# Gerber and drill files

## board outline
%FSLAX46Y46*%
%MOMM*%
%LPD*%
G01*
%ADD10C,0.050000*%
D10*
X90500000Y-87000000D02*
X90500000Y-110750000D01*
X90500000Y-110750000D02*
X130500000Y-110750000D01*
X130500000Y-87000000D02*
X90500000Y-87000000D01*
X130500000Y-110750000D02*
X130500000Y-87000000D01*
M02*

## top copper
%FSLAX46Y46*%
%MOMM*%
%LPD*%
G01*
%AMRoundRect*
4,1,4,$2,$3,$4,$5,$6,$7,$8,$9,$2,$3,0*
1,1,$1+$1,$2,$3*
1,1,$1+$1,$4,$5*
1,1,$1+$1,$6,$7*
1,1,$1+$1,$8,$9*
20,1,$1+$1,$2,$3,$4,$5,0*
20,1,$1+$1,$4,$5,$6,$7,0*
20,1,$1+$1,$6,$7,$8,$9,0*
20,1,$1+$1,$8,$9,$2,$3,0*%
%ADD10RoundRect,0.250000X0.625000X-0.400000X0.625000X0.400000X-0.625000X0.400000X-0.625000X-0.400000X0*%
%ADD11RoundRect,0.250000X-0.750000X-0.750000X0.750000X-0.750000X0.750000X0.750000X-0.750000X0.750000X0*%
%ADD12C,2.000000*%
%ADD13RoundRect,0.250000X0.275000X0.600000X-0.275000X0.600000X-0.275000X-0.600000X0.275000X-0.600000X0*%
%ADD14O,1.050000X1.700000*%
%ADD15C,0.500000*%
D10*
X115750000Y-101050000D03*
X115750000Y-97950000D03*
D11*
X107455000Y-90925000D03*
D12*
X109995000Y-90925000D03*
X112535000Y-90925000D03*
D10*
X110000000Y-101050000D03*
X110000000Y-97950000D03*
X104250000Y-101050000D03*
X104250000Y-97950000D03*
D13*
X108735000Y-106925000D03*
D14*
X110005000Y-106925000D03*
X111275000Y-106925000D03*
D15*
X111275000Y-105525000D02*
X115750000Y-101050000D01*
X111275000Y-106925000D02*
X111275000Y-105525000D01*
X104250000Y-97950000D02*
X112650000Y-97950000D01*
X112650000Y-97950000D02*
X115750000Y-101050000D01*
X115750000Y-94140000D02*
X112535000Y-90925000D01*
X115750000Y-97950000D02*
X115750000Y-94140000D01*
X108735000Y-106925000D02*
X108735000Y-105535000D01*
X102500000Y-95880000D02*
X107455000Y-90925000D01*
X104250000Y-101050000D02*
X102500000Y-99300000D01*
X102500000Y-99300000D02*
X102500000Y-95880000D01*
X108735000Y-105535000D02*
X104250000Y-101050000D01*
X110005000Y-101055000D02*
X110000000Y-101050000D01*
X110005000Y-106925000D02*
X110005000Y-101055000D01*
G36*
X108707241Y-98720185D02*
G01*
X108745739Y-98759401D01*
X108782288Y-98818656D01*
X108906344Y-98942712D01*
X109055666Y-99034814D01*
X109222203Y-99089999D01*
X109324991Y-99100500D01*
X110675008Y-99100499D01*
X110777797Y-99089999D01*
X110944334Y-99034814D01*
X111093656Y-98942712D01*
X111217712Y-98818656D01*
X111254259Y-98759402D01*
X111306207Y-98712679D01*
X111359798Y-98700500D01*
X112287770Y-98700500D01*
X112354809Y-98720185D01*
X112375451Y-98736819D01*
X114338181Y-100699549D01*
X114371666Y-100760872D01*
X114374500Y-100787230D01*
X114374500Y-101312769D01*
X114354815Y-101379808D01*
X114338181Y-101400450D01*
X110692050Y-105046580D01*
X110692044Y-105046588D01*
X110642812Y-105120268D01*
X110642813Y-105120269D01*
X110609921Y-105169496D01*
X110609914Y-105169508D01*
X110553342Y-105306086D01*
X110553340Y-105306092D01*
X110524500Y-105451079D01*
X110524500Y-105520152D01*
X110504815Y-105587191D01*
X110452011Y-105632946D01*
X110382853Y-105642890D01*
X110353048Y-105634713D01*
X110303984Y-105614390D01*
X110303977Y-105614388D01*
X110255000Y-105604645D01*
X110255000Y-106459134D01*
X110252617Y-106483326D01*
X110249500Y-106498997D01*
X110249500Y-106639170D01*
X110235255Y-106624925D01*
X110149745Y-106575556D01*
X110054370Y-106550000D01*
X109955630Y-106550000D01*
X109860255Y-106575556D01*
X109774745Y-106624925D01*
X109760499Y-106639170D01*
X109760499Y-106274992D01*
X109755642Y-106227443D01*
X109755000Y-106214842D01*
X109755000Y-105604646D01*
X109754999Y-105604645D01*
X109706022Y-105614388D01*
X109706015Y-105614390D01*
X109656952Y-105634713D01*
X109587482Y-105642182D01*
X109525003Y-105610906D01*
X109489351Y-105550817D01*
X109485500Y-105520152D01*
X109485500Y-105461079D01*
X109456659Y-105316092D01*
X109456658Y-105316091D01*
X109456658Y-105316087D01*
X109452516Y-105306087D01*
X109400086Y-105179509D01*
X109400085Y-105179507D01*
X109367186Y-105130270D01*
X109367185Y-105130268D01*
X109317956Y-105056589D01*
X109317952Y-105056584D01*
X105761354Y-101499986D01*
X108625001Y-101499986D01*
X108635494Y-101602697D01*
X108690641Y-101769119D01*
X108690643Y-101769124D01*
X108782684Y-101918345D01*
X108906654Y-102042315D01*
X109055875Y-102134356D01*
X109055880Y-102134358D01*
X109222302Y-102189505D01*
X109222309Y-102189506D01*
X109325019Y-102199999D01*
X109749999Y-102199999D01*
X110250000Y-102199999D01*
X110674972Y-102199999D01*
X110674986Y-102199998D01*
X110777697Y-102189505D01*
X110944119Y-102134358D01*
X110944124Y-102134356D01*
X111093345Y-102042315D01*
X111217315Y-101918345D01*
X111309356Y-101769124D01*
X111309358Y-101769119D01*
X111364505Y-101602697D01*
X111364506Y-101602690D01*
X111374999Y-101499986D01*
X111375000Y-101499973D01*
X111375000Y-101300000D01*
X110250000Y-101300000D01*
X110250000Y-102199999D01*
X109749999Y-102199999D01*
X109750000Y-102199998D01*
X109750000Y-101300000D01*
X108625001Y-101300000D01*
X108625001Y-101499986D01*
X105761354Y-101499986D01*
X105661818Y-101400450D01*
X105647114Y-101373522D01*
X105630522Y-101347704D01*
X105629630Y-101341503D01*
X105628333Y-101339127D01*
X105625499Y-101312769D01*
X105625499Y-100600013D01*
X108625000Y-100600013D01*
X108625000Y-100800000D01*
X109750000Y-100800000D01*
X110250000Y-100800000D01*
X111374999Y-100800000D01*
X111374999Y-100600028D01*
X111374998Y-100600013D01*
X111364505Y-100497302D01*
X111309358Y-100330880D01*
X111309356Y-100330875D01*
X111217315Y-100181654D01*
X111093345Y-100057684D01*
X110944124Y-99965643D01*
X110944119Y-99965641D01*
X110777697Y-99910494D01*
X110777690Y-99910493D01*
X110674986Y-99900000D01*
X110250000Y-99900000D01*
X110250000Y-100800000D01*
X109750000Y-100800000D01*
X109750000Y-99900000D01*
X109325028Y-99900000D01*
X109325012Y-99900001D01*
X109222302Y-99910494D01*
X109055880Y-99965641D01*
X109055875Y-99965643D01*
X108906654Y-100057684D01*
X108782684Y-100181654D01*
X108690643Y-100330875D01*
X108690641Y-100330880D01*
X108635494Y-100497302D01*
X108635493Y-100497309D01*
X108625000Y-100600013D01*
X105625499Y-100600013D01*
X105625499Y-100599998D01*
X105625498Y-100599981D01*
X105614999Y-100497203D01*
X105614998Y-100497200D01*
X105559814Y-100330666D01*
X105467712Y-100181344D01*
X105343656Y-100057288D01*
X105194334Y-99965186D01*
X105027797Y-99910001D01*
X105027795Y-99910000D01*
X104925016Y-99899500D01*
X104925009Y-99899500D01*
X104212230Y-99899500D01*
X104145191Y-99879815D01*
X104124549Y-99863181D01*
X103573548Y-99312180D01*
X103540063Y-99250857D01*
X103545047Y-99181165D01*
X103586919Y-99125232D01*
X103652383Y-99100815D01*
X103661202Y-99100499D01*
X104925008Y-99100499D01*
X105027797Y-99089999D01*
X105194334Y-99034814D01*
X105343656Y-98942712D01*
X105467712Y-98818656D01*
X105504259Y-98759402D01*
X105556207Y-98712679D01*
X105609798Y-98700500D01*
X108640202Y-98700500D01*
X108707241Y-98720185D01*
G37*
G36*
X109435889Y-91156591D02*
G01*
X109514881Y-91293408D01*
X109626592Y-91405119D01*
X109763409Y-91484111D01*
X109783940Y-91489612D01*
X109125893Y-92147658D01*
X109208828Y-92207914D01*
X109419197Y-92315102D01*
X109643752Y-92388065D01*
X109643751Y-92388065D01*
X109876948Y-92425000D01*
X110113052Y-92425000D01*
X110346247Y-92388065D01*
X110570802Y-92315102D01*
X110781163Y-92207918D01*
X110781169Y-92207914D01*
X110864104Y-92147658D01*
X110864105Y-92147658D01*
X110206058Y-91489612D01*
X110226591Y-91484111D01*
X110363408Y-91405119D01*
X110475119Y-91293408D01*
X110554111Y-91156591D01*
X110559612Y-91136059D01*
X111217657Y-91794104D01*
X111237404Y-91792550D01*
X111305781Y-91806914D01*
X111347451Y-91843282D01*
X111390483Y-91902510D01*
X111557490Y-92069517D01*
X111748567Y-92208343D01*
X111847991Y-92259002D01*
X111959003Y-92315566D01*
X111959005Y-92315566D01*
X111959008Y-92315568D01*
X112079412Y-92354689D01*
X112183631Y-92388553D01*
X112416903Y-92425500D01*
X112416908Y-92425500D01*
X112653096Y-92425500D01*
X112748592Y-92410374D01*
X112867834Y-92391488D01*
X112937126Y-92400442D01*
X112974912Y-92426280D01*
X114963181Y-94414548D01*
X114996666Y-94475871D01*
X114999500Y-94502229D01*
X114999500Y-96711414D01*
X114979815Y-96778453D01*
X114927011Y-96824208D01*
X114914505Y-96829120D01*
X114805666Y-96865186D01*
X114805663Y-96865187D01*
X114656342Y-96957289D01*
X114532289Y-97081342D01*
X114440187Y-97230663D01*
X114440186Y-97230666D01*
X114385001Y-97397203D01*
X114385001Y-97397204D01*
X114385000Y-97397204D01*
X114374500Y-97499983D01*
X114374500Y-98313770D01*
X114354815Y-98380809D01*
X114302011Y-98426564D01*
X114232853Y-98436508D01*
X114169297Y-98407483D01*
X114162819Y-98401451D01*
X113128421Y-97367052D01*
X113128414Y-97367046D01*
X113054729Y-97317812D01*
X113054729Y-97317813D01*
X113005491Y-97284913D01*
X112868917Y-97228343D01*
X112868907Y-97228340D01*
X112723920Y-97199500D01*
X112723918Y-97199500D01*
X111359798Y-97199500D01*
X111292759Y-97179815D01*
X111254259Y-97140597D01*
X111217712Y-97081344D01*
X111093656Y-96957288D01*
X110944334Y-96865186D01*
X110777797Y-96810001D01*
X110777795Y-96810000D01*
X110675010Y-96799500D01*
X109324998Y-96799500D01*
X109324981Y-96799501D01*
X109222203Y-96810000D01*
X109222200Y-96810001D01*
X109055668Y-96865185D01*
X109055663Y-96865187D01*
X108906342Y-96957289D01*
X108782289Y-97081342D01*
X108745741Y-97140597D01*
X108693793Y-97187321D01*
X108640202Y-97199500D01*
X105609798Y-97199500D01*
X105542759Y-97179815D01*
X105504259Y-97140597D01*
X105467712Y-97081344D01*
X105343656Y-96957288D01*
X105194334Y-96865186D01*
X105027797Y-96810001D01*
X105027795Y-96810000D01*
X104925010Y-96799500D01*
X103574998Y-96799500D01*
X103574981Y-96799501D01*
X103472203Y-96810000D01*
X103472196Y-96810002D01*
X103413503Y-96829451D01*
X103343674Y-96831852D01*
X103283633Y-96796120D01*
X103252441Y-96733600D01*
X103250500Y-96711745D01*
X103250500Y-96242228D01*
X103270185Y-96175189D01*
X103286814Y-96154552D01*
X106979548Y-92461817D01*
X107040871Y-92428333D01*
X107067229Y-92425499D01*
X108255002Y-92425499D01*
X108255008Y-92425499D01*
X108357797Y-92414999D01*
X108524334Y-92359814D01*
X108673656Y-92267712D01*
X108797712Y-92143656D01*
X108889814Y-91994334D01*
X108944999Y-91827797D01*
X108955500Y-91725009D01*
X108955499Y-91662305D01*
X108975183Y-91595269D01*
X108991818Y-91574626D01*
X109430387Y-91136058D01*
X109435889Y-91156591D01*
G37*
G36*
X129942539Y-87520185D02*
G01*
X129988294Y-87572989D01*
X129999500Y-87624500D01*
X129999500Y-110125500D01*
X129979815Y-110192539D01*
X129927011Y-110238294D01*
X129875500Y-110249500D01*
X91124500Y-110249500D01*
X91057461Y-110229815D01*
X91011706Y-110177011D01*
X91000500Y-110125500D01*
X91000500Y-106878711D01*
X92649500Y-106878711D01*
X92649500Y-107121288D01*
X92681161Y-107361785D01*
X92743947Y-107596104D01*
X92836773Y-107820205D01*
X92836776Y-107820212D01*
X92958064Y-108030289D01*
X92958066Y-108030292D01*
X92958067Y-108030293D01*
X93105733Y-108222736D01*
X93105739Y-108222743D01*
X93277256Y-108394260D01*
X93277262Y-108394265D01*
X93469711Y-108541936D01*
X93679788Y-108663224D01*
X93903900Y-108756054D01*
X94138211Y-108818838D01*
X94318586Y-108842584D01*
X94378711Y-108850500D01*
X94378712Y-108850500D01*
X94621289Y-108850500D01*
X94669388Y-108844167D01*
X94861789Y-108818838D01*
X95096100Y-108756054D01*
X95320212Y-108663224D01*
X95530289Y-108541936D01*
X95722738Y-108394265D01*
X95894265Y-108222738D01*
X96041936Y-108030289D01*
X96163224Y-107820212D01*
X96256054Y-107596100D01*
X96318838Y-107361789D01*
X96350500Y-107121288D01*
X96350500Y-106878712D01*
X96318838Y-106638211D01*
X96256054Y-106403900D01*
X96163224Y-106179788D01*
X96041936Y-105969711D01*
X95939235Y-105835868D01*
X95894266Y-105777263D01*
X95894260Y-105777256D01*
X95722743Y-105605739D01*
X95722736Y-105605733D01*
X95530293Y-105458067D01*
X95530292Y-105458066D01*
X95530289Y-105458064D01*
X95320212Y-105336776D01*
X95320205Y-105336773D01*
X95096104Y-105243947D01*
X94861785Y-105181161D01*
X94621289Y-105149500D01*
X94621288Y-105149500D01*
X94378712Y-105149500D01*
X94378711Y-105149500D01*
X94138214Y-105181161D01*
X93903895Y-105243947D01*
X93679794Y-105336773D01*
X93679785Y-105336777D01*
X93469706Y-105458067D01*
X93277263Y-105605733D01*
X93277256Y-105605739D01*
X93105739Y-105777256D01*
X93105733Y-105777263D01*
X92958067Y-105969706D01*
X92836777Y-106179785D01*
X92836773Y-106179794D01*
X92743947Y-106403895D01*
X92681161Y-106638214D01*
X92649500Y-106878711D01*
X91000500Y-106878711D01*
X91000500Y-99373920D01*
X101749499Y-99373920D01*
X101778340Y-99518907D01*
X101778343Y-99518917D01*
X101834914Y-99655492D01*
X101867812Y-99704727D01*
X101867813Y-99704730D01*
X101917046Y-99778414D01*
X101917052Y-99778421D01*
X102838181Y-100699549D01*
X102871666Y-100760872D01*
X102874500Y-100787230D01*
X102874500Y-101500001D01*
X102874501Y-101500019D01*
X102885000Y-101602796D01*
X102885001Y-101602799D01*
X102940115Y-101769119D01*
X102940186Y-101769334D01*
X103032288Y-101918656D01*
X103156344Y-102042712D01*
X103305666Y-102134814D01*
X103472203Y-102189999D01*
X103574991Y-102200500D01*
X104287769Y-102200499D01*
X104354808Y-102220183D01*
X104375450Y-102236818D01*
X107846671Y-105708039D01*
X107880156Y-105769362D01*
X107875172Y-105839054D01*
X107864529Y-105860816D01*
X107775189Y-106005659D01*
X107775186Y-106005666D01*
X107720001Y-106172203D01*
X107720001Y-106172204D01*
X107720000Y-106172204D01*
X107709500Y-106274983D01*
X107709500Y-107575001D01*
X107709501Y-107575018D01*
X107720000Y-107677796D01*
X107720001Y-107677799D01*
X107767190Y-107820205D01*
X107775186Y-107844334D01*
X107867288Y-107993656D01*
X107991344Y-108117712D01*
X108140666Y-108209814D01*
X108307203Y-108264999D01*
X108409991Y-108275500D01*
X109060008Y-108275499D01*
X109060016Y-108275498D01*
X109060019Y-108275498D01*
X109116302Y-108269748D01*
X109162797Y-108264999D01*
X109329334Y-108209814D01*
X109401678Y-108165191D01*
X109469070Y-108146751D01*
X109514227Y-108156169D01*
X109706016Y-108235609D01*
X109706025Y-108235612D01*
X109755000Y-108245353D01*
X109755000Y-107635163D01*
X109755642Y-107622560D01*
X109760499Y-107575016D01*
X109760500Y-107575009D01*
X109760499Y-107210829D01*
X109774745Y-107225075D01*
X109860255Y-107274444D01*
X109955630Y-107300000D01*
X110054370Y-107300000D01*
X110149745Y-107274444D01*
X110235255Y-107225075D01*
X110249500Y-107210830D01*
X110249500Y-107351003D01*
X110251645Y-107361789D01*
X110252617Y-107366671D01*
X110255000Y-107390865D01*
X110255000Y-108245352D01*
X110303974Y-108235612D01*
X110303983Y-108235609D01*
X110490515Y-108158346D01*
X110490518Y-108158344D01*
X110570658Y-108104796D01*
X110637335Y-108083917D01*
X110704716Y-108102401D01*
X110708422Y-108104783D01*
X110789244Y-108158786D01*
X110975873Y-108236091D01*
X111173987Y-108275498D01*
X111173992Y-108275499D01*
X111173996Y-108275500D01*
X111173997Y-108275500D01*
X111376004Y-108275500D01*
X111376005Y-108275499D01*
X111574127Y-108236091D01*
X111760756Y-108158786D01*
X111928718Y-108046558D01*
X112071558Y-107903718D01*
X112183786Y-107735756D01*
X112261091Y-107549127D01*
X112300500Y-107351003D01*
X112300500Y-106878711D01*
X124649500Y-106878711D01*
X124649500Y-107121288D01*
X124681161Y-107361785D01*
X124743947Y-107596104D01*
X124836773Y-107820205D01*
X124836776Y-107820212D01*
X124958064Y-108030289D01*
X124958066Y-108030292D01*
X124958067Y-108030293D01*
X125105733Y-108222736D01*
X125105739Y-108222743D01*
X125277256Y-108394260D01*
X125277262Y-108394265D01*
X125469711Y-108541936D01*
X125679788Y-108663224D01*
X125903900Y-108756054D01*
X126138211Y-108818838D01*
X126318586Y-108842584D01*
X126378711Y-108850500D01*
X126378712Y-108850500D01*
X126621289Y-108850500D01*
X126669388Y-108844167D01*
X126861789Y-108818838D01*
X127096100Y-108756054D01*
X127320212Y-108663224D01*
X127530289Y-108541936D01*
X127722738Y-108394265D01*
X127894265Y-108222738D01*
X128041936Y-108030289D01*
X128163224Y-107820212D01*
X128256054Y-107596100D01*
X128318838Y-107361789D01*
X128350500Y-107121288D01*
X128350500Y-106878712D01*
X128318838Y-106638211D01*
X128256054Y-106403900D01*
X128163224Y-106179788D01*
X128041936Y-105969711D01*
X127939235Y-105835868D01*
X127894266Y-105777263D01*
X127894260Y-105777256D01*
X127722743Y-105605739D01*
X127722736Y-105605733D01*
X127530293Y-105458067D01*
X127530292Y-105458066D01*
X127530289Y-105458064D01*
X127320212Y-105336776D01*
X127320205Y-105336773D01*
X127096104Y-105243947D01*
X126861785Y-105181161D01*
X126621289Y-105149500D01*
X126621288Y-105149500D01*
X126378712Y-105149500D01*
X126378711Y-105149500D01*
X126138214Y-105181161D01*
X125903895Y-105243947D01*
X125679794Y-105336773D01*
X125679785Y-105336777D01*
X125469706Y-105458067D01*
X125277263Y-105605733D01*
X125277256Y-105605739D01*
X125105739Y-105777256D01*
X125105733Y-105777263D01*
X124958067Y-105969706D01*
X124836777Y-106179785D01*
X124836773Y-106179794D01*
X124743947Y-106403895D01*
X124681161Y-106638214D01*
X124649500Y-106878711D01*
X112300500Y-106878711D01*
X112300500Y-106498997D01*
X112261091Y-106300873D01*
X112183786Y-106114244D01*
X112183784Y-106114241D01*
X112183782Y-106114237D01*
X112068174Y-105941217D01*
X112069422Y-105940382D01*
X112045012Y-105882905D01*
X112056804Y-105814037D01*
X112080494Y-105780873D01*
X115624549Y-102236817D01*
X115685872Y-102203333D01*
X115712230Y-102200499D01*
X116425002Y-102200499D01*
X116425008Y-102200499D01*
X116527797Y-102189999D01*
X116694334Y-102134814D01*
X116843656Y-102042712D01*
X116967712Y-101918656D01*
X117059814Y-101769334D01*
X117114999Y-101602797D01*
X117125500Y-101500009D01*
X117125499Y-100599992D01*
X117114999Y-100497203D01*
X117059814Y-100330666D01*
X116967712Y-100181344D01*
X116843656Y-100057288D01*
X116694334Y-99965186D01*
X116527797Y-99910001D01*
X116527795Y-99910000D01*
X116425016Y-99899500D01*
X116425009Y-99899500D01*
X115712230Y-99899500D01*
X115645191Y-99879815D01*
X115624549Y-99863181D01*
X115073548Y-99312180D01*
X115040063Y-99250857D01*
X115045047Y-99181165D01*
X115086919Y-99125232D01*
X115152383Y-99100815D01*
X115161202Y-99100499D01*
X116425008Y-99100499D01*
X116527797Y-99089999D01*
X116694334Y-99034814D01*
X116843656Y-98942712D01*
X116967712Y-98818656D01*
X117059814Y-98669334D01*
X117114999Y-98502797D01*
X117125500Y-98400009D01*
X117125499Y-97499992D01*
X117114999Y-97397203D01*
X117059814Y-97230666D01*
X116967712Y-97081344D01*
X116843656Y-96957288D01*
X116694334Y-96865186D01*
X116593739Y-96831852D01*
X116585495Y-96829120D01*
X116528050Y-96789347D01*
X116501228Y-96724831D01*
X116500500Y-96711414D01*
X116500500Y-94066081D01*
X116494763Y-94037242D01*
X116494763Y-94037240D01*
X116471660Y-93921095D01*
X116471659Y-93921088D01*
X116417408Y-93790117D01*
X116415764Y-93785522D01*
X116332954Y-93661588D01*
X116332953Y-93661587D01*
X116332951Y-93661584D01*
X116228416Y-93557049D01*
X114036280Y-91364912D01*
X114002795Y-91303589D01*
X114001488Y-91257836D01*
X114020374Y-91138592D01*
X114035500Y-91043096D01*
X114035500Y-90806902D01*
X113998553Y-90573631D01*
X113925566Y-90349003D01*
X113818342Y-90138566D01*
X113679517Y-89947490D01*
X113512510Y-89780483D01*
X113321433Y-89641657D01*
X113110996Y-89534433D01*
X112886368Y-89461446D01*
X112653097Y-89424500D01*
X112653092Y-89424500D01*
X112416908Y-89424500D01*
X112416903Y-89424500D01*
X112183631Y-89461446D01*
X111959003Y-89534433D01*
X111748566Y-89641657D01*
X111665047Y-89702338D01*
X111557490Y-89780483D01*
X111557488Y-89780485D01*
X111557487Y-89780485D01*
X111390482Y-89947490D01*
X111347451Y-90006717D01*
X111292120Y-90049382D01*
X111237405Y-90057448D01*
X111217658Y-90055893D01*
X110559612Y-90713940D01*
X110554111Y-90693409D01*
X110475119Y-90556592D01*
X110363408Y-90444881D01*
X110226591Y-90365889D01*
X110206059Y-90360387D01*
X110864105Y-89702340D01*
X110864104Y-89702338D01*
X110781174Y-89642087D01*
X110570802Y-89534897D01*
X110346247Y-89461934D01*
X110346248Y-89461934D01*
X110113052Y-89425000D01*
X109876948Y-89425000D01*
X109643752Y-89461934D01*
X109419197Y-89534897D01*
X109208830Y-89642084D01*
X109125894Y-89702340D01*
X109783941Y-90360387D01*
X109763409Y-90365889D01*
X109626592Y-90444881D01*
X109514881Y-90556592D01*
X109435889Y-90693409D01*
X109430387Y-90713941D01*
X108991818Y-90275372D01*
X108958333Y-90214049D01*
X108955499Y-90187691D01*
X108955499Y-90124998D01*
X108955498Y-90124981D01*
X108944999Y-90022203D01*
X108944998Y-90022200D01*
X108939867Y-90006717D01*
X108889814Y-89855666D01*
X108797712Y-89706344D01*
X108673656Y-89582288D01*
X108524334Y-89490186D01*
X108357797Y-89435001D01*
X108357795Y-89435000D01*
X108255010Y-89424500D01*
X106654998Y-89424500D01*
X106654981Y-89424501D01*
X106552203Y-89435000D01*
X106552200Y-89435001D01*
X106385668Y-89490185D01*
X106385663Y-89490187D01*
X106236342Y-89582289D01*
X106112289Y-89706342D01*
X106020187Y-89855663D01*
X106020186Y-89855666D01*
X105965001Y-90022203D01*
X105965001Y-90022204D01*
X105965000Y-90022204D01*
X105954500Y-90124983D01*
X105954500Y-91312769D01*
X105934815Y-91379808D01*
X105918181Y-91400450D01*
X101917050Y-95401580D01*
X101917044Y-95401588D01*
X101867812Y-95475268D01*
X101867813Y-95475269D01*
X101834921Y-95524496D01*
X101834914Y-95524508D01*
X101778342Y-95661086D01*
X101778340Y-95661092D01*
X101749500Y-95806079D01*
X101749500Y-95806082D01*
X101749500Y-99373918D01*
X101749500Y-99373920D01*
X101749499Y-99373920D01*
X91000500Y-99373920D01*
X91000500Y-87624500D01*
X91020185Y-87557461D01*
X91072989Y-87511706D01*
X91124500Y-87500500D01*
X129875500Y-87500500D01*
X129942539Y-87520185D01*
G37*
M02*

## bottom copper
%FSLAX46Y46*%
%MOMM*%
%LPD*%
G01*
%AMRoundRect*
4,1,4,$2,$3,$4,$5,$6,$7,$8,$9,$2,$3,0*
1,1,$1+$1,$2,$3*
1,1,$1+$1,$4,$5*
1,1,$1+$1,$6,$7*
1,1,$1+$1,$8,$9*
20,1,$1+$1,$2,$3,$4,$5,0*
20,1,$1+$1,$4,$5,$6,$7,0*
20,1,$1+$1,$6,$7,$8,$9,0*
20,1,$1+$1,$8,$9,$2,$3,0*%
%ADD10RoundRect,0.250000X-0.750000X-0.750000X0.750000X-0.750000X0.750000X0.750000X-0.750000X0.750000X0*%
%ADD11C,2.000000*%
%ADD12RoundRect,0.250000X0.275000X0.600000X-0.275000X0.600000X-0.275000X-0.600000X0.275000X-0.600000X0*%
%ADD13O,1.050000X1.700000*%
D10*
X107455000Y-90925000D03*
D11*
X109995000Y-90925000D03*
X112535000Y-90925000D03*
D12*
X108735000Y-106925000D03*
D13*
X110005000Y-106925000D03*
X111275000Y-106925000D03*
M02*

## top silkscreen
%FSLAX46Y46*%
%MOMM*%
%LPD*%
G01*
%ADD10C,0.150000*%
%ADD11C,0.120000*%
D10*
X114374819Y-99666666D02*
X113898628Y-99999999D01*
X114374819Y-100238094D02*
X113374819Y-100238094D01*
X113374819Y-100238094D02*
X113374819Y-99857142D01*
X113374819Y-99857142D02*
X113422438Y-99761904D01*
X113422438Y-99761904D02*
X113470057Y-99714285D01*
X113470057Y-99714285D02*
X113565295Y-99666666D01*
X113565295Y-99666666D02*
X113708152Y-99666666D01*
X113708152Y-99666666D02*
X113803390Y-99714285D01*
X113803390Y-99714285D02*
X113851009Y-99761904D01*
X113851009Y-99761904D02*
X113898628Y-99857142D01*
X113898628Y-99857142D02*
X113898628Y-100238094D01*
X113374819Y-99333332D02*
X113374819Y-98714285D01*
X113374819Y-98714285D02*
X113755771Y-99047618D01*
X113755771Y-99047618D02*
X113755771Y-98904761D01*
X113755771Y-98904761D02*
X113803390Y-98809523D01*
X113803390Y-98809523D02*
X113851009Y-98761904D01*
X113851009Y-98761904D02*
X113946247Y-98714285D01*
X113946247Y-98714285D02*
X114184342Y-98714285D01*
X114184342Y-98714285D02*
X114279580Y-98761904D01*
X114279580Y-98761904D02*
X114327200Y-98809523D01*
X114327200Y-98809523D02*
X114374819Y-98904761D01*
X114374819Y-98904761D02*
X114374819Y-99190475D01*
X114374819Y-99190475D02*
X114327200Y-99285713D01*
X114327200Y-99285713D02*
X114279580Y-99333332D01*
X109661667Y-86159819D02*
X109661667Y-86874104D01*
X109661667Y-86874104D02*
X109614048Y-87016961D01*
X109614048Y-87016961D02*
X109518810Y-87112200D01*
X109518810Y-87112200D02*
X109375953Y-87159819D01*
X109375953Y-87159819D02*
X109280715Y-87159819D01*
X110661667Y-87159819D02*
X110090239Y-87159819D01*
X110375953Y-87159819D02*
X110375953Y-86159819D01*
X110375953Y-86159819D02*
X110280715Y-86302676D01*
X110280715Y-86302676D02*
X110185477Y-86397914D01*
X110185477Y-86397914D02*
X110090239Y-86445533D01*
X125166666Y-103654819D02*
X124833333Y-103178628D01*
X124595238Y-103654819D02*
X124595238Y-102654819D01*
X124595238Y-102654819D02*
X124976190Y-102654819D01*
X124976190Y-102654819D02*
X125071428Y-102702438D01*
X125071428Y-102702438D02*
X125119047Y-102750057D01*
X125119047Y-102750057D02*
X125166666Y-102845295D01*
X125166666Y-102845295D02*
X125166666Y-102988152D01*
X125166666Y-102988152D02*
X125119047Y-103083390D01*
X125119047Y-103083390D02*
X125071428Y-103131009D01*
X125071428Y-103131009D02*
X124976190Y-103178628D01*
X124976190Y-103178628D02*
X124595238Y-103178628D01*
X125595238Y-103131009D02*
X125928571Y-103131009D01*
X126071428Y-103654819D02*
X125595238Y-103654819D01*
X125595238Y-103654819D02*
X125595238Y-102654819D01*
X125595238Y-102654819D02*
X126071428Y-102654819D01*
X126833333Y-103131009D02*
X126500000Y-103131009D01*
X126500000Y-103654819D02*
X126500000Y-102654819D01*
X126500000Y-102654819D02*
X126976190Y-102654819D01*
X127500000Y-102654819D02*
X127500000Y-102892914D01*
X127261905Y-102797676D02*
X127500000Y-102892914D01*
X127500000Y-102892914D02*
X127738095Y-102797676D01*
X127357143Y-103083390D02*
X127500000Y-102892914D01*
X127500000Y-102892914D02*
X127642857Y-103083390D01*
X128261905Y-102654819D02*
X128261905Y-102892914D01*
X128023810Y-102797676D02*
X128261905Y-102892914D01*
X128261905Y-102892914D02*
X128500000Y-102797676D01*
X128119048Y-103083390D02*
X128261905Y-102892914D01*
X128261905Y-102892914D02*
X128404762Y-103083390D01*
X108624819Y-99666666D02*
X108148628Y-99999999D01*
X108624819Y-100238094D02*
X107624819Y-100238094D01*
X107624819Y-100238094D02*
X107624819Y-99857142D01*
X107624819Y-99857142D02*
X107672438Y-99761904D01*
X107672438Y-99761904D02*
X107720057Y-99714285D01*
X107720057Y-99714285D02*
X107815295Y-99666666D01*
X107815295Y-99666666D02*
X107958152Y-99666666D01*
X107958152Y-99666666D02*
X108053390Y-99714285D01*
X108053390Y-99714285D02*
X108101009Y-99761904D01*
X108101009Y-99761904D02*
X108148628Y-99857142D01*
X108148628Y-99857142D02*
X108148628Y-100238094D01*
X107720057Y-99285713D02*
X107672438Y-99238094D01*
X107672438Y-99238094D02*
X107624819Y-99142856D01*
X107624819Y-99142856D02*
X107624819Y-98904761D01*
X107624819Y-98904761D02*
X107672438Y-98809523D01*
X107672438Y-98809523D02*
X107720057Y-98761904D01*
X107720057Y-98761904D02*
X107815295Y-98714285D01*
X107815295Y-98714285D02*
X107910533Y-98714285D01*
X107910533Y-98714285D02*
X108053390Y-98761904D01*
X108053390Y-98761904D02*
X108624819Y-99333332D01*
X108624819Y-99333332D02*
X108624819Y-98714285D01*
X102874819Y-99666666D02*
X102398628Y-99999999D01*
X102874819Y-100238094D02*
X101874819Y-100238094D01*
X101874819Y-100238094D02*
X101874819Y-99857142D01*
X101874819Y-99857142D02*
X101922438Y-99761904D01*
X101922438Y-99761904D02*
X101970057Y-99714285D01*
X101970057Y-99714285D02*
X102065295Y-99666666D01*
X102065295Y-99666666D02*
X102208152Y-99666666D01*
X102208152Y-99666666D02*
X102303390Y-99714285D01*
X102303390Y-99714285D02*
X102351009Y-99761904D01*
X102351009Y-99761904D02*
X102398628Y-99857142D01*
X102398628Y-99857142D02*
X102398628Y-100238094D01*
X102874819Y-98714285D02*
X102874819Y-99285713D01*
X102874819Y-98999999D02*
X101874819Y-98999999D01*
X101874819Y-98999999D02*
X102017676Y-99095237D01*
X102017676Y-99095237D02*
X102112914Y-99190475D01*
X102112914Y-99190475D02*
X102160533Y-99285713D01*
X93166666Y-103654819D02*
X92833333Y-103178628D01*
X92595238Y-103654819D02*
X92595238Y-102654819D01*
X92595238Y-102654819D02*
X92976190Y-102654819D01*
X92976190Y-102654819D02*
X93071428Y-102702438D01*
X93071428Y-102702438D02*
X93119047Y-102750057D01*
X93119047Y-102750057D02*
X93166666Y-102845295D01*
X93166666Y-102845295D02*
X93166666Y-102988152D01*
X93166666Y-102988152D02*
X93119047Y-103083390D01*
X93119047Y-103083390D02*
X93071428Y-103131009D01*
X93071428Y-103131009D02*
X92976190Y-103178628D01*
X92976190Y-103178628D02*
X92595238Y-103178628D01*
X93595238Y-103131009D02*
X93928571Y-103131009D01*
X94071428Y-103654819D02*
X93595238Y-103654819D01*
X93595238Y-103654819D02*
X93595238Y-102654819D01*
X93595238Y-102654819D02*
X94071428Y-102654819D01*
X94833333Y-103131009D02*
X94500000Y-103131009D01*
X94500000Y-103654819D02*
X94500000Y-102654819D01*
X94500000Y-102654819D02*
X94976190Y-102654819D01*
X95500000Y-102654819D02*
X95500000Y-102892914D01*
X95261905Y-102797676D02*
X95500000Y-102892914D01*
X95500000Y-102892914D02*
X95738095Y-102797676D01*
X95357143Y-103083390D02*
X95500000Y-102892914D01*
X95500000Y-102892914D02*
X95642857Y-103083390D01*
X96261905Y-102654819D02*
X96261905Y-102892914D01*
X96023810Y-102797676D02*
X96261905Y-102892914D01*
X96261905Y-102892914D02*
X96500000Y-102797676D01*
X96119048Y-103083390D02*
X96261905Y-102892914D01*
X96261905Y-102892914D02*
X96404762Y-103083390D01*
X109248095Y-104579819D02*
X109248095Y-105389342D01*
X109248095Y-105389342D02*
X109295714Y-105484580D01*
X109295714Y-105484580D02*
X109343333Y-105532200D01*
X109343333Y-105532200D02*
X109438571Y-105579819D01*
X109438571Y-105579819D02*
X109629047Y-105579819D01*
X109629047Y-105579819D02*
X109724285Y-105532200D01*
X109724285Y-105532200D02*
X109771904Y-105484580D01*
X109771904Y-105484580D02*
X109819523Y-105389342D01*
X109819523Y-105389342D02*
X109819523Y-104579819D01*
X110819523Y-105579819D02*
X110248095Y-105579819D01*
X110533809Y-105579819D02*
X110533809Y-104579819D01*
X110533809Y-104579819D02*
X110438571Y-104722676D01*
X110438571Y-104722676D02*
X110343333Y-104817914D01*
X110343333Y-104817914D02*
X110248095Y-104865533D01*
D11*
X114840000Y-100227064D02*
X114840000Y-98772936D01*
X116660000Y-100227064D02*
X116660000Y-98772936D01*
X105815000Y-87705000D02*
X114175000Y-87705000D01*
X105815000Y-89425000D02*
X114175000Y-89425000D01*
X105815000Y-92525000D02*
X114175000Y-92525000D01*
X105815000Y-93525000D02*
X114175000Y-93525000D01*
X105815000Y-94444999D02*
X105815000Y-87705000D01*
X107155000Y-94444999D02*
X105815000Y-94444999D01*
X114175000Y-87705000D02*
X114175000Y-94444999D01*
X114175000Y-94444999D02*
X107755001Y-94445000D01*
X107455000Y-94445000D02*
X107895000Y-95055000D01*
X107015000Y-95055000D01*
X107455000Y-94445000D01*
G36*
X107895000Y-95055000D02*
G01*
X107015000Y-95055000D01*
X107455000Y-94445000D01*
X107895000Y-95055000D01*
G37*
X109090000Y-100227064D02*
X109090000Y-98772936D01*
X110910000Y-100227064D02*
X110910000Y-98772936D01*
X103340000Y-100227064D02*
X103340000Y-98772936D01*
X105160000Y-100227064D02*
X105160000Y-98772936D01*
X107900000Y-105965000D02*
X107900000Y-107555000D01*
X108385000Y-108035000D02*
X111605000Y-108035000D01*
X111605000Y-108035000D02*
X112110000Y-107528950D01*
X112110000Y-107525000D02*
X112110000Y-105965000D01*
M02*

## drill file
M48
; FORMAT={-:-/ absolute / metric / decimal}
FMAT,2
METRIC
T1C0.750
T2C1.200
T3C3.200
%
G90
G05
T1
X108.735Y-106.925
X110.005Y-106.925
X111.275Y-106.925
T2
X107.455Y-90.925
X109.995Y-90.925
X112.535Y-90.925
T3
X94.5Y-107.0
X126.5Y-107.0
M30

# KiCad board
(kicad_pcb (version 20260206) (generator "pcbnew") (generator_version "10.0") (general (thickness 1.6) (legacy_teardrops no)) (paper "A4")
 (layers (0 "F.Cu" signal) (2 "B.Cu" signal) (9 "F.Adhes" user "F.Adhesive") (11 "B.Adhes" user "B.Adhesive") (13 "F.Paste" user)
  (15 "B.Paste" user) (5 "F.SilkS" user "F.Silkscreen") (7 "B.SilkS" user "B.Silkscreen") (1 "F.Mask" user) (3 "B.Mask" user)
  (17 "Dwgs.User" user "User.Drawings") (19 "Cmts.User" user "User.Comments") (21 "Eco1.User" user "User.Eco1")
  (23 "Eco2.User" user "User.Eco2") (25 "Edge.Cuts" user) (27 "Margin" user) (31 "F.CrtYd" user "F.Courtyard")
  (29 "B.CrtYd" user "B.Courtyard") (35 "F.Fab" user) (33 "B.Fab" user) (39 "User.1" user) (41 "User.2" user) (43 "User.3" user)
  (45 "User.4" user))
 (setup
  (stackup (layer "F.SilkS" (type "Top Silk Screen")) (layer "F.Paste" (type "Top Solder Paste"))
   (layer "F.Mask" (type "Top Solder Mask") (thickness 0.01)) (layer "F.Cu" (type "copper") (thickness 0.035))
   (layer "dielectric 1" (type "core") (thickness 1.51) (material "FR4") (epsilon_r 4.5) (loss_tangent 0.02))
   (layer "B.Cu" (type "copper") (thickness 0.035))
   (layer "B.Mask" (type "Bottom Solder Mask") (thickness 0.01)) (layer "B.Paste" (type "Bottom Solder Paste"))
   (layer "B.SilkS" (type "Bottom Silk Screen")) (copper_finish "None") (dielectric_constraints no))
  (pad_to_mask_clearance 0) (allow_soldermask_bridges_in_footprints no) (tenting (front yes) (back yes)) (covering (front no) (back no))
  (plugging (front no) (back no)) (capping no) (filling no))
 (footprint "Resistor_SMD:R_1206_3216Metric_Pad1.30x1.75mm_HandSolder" (layer "F.Cu") (at 115.75 99.5 90)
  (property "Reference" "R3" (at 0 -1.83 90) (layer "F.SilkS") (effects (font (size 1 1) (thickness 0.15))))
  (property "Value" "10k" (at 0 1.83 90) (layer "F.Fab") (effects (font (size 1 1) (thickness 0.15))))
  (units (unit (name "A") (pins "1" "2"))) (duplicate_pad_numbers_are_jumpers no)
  (fp_line (start -0.727064 -0.91) (end 0.727064 -0.91) (stroke (width 0.12) (type solid)) (layer "F.SilkS"))
  (fp_line (start -0.727064 0.91) (end 0.727064 0.91) (stroke (width 0.12) (type solid)) (layer "F.SilkS"))
  (pad "1" smd roundrect (at -1.55 0 90) (size 1.3 1.75) (layers "F.Cu" "F.Mask" "F.Paste") (roundrect_rratio 0.192308)
   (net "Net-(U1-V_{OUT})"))
  (pad "2" smd roundrect (at 1.55 0 90) (size 1.3 1.75) (layers "F.Cu" "F.Mask" "F.Paste") (roundrect_rratio 0.192308) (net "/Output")))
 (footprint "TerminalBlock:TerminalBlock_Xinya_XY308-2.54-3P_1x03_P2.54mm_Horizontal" (layer "F.Cu") (at 107.455 90.925)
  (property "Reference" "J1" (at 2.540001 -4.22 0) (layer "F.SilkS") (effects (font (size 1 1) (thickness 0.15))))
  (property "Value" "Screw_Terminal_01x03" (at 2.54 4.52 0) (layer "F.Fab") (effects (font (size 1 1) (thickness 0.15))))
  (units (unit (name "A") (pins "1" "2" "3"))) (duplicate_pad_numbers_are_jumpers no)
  (fp_line (start -1.64 -3.22) (end 6.72 -3.22) (stroke (width 0.12) (type solid)) (layer "F.SilkS"))
  (fp_line (start -1.64 -1.5) (end 6.72 -1.5) (stroke (width 0.12) (type solid)) (layer "F.SilkS"))
  (fp_line (start -1.64 1.6) (end 6.72 1.6) (stroke (width 0.12) (type solid)) (layer "F.SilkS"))
  (fp_line (start -1.64 2.6) (end 6.72 2.6) (stroke (width 0.12) (type solid)) (layer "F.SilkS"))
  (fp_line (start -1.64 3.519999) (end -1.64 -3.22) (stroke (width 0.12) (type solid)) (layer "F.SilkS"))
  (fp_line (start -0.3 3.519999) (end -1.64 3.519999) (stroke (width 0.12) (type solid)) (layer "F.SilkS"))
  (fp_line (start 6.72 -3.22) (end 6.72 3.519999) (stroke (width 0.12) (type solid)) (layer "F.SilkS"))
  (fp_line (start 6.72 3.519999) (end 0.300001 3.52) (stroke (width 0.12) (type solid)) (layer "F.SilkS"))
  (fp_poly (pts (xy 0 3.52) (xy 0.44 4.13) (xy -0.44 4.13)) (stroke (width 0.12) (type solid)) (fill yes) (layer "F.SilkS"))
  (pad "1" thru_hole roundrect (at 0 0) (size 2 2) (drill 1.2) (layers "*.Cu" "*.Mask") (remove_unused_layers no) (roundrect_rratio 0.125)
   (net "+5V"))
  (pad "2" thru_hole circle (at 2.54 0) (size 2 2) (drill 1.2) (layers "*.Cu" "*.Mask") (remove_unused_layers no) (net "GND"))
  (pad "3" thru_hole circle (at 5.08 0) (size 2 2) (drill 1.2) (layers "*.Cu" "*.Mask") (remove_unused_layers no) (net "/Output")))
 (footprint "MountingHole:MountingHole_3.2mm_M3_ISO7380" (layer "F.Cu") (at 126.5 107)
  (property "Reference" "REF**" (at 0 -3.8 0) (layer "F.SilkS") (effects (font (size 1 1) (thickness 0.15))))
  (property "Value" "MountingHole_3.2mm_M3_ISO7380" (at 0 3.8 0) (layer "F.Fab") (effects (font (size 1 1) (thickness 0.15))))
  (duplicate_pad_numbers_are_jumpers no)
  (pad "" np_thru_hole circle (at 0 0) (size 3.2 3.2) (drill 3.2) (layers "*.Cu" "*.Mask")))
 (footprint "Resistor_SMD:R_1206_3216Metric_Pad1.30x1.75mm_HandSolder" (layer "F.Cu") (at 110 99.5 90)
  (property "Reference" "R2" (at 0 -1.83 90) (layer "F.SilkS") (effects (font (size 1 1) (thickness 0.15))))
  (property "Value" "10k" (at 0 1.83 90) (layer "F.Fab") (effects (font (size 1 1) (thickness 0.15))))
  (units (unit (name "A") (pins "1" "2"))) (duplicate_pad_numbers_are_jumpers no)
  (fp_line (start -0.727064 -0.91) (end 0.727064 -0.91) (stroke (width 0.12) (type solid)) (layer "F.SilkS"))
  (fp_line (start -0.727064 0.91) (end 0.727064 0.91) (stroke (width 0.12) (type solid)) (layer "F.SilkS"))
  (pad "1" smd roundrect (at -1.55 0 90) (size 1.3 1.75) (layers "F.Cu" "F.Mask" "F.Paste") (roundrect_rratio 0.192308) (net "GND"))
  (pad "2" smd roundrect (at 1.55 0 90) (size 1.3 1.75) (layers "F.Cu" "F.Mask" "F.Paste") (roundrect_rratio 0.192308)
   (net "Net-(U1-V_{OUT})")))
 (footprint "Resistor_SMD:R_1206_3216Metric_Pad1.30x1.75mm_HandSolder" (layer "F.Cu") (at 104.25 99.5 90)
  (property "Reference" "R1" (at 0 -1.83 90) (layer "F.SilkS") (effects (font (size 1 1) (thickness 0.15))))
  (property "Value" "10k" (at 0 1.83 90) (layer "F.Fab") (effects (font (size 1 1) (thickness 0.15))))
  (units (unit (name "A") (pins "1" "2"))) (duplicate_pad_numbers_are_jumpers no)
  (fp_line (start -0.727064 -0.91) (end 0.727064 -0.91) (stroke (width 0.12) (type solid)) (layer "F.SilkS"))
  (fp_line (start -0.727064 0.91) (end 0.727064 0.91) (stroke (width 0.12) (type solid)) (layer "F.SilkS"))
  (pad "1" smd roundrect (at -1.55 0 90) (size 1.3 1.75) (layers "F.Cu" "F.Mask" "F.Paste") (roundrect_rratio 0.192308) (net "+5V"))
  (pad "2" smd roundrect (at 1.55 0 90) (size 1.3 1.75) (layers "F.Cu" "F.Mask" "F.Paste") (roundrect_rratio 0.192308)
   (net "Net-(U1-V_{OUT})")))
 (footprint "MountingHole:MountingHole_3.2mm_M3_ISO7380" (layer "F.Cu") (at 94.5 107)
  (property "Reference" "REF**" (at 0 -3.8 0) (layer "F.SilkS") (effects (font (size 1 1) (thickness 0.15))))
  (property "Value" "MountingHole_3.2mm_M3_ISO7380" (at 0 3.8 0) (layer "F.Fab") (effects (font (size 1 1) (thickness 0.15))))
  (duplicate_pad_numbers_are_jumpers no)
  (pad "" np_thru_hole circle (at 0 0) (size 3.2 3.2) (drill 3.2) (layers "*.Cu" "*.Mask")))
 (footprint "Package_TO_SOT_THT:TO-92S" (layer "F.Cu") (at 108.735 106.925)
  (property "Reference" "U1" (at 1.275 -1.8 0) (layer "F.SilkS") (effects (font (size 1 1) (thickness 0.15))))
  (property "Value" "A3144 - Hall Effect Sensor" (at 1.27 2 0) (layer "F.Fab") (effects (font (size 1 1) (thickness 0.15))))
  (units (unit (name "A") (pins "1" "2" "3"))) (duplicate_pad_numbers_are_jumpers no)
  (fp_line (start -0.835 -0.96) (end -0.835 0.63) (stroke (width 0.12) (type solid)) (layer "F.SilkS"))
  (fp_line (start -0.35 1.11) (end 2.87 1.11) (stroke (width 0.12) (type solid)) (layer "F.SilkS"))
  (fp_line (start 2.87 1.11) (end 3.375 0.60395) (stroke (width 0.12) (type solid)) (layer "F.SilkS"))
  (fp_line (start 3.375 0.6) (end 3.375 -0.96) (stroke (width 0.12) (type solid)) (layer "F.SilkS"))
  (pad "1" thru_hole roundrect (at 0 0 180) (size 1.05 1.7) (drill 0.75) (layers "*.Cu" "*.Mask") (remove_unused_layers no)
   (roundrect_rratio 0.2380952381) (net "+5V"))
  (pad "2" thru_hole oval (at 1.27 0 180) (size 1.05 1.7) (drill 0.75) (layers "*.Cu" "*.Mask") (remove_unused_layers no) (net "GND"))
  (pad "3" thru_hole oval (at 2.54 0 180) (size 1.05 1.7) (drill 0.75) (layers "*.Cu" "*.Mask") (remove_unused_layers no)
   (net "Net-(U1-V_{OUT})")))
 (gr_line (start 90.5 87) (end 90.5 110.75) (stroke (width 0.05) (type default)) (layer "Edge.Cuts"))
 (gr_line (start 90.5 110.75) (end 130.5 110.75) (stroke (width 0.05) (type default)) (layer "Edge.Cuts"))
 (gr_line (start 130.5 87) (end 90.5 87) (stroke (width 0.05) (type default)) (layer "Edge.Cuts"))
 (gr_line (start 130.5 110.75) (end 130.5 87) (stroke (width 0.05) (type default)) (layer "Edge.Cuts"))
 (segment (start 111.275 105.525) (end 115.75 101.05) (width 0.5) (layer "F.Cu") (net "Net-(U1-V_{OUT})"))
 (segment (start 111.275 106.925) (end 111.275 105.525) (width 0.5) (layer "F.Cu") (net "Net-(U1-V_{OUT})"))
 (segment (start 104.25 97.95) (end 112.65 97.95) (width 0.5) (layer "F.Cu") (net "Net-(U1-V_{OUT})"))
 (segment (start 112.65 97.95) (end 115.75 101.05) (width 0.5) (layer "F.Cu") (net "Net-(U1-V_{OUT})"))
 (segment (start 115.75 94.14) (end 112.535 90.925) (width 0.5) (layer "F.Cu") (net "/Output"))
 (segment (start 115.75 97.95) (end 115.75 94.14) (width 0.5) (layer "F.Cu") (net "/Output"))
 (segment (start 108.735 106.925) (end 108.735 105.535) (width 0.5) (layer "F.Cu") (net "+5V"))
 (segment (start 102.5 95.88) (end 107.455 90.925) (width 0.5) (layer "F.Cu") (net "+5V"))
 (segment (start 104.25 101.05) (end 102.5 99.3) (width 0.5) (layer "F.Cu") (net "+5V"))
 (segment (start 102.5 99.3) (end 102.5 95.88) (width 0.5) (layer "F.Cu") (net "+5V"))
 (segment (start 108.735 105.535) (end 104.25 101.05) (width 0.5) (layer "F.Cu") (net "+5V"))
 (segment (start 110.005 101.055) (end 110 101.05) (width 0.5) (layer "F.Cu") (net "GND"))
 (segment (start 110.005 106.925) (end 110.005 101.055) (width 0.5) (layer "F.Cu") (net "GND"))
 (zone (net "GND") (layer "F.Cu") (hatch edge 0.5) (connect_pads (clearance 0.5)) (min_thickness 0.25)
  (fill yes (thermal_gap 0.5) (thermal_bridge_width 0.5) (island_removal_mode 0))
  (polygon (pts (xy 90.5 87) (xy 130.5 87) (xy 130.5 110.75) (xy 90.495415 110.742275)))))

